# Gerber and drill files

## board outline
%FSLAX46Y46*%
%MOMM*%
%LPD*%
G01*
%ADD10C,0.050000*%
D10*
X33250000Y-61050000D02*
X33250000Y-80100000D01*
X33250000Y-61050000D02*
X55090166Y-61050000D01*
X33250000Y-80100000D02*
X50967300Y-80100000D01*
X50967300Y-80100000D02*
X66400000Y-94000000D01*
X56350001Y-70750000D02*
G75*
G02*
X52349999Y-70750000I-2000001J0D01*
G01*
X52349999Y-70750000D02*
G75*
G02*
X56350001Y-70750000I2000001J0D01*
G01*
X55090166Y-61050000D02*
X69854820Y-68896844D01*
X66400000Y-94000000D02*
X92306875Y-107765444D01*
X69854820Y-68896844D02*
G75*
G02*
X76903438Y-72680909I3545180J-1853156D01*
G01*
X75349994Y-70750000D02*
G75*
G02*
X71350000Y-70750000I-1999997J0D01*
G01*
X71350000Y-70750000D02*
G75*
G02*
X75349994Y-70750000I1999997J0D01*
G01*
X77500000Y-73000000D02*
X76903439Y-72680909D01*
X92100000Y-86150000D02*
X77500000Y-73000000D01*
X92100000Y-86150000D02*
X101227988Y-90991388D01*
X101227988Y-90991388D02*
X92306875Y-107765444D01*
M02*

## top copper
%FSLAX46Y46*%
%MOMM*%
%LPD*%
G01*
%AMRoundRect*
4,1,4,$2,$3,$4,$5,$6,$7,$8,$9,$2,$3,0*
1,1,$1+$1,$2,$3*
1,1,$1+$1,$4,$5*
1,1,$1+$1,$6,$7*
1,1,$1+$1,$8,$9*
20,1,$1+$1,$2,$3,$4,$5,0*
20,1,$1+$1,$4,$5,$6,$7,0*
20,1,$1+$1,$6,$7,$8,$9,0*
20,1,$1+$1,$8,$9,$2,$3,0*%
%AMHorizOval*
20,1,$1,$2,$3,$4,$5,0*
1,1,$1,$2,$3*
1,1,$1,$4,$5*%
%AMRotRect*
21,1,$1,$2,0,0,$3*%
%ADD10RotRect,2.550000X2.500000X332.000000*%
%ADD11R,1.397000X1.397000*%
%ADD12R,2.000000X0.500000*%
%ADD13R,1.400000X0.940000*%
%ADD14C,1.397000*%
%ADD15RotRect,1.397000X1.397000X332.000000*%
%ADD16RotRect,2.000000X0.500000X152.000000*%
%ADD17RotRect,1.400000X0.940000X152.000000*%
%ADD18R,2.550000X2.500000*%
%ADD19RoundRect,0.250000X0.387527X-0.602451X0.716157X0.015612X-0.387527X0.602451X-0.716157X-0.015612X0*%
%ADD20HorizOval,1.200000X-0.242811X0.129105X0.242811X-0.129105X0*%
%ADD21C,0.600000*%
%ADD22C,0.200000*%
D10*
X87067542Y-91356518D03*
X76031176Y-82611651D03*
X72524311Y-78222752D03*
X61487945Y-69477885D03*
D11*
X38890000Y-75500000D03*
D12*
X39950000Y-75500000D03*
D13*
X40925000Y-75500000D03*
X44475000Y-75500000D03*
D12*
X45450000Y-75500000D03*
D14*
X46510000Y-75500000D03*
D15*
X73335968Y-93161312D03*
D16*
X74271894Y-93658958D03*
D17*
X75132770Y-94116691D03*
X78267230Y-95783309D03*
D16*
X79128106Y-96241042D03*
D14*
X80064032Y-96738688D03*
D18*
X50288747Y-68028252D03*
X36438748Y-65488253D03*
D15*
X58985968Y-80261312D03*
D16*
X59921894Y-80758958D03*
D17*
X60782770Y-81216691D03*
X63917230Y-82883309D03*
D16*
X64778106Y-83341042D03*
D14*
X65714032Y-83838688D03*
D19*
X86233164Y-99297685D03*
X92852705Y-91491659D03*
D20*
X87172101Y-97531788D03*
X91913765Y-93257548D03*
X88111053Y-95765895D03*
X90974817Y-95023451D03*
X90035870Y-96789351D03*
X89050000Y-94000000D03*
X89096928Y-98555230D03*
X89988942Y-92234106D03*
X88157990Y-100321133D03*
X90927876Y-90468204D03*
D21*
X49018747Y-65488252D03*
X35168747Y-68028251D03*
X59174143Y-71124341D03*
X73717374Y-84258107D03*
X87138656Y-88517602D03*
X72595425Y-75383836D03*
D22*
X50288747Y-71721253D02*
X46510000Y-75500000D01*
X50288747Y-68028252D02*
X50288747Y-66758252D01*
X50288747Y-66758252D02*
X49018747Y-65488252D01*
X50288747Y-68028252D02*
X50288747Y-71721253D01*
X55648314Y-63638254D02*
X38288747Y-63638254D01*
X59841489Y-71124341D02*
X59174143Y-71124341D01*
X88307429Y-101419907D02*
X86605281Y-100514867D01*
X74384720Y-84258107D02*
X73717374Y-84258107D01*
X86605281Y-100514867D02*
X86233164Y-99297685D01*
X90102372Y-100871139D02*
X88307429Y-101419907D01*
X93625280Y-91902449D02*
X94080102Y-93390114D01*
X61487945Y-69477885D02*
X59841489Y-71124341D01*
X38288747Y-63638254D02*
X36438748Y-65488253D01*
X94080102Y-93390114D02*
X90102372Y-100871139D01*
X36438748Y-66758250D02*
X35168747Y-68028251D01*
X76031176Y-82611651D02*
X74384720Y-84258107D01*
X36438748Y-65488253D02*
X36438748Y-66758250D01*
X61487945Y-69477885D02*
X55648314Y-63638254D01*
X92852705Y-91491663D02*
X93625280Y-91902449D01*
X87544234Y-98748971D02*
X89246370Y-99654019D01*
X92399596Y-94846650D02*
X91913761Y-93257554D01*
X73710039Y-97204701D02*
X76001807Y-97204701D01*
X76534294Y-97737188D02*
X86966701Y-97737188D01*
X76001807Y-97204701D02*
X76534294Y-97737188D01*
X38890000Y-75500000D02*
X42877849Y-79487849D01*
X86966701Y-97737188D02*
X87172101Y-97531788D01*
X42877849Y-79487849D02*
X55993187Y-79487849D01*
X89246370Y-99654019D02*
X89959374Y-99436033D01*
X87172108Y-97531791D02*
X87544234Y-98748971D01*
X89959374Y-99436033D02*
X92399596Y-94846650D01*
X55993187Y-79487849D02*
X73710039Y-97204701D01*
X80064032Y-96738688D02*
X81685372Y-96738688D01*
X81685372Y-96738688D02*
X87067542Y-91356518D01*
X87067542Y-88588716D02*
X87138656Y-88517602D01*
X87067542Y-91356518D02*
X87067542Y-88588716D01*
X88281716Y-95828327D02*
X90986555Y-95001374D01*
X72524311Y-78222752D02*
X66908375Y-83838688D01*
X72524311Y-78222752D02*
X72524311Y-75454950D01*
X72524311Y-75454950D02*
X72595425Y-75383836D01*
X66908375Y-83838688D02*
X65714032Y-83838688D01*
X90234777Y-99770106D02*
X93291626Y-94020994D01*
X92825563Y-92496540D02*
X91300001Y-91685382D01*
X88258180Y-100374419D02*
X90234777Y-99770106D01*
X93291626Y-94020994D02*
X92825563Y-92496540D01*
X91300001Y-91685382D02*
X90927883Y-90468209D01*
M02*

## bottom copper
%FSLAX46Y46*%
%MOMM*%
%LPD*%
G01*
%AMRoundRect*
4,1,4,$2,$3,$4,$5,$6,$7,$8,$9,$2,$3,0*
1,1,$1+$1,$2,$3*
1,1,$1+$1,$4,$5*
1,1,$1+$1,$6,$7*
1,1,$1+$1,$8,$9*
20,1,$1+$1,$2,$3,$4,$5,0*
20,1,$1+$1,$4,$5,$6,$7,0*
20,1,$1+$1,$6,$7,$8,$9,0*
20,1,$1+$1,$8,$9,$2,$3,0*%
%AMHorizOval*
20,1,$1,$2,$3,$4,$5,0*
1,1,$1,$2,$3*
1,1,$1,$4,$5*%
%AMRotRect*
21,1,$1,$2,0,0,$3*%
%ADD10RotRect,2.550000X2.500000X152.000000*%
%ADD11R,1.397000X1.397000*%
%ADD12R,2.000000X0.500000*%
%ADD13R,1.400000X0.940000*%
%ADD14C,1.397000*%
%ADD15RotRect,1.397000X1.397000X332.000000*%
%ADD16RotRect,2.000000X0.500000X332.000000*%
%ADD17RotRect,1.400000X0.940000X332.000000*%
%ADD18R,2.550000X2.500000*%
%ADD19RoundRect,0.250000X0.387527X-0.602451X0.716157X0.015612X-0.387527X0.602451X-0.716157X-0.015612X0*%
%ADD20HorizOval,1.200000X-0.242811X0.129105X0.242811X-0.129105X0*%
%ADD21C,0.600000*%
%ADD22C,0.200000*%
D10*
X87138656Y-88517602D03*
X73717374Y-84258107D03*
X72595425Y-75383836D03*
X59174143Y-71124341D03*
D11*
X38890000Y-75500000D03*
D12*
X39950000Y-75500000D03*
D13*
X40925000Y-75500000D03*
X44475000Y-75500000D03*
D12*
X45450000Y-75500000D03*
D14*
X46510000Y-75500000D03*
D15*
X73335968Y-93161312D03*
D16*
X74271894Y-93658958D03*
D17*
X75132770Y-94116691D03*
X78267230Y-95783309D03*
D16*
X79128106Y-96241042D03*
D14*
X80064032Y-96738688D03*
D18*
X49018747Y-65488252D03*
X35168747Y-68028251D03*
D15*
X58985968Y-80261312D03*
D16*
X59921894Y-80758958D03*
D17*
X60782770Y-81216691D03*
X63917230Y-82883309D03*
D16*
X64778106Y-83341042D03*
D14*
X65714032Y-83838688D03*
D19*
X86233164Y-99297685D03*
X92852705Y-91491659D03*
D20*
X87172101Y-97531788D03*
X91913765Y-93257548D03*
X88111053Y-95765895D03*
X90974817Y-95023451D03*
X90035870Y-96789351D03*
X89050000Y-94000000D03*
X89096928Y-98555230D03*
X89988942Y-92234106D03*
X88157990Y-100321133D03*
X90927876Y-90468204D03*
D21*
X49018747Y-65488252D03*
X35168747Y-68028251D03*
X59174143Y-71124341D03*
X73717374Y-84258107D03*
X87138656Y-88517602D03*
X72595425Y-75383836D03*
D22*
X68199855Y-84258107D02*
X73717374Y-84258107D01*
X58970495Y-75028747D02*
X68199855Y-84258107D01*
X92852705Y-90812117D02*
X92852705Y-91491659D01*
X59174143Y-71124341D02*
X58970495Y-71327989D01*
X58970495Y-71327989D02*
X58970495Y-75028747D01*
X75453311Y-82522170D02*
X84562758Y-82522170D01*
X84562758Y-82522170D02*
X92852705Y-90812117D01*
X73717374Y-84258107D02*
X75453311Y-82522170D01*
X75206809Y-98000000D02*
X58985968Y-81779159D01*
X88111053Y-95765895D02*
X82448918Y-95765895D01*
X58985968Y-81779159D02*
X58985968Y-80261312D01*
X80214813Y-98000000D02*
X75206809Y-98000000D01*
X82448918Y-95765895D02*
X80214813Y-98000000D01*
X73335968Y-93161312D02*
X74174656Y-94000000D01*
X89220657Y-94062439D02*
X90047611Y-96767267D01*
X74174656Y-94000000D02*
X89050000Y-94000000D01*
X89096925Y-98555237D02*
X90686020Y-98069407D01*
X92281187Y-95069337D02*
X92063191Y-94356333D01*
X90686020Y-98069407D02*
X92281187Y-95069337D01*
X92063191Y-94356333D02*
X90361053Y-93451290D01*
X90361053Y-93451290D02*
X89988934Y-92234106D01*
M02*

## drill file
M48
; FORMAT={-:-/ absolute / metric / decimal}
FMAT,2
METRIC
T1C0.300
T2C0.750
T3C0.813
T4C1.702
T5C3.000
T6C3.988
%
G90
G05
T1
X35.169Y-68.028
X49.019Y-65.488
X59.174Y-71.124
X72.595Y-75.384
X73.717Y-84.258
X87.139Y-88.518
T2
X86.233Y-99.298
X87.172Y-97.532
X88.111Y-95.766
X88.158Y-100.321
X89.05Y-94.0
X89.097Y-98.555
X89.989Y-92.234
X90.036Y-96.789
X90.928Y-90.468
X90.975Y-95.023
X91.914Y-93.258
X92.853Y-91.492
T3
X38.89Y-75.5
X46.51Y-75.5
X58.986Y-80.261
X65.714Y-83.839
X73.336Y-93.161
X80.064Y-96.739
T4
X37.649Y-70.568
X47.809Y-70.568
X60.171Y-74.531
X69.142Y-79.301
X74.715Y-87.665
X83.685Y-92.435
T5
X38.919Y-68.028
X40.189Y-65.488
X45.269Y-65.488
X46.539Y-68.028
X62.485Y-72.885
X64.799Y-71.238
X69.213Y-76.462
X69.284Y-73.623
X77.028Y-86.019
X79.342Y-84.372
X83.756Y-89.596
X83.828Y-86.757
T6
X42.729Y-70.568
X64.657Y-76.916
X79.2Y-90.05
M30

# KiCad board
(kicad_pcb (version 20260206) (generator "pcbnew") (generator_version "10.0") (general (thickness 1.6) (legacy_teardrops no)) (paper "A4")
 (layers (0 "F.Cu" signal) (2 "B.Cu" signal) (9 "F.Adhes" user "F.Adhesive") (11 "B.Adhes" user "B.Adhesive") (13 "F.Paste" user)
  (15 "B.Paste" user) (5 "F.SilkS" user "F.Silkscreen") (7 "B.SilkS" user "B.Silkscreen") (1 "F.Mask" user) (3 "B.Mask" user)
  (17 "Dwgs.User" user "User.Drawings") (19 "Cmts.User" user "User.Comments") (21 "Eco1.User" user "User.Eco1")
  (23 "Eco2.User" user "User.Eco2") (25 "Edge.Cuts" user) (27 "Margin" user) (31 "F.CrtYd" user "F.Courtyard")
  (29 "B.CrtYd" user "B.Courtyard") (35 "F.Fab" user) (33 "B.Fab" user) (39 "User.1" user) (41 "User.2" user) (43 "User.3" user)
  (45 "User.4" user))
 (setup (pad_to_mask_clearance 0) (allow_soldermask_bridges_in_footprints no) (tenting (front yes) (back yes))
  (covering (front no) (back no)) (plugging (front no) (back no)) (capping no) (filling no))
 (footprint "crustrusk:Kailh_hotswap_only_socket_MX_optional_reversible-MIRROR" (layer "F.Cu") (at 79.2 90.05 -28)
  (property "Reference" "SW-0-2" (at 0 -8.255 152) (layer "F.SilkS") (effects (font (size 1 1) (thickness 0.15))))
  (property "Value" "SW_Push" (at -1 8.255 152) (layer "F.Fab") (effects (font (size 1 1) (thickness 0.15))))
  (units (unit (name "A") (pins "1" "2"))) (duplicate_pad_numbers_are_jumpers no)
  (pad "" np_thru_hole circle (at -5.08 0 332) (size 1.7018 1.7018) (drill 1.7018) (layers "*.Cu" "*.Mask"))
  (pad "" np_thru_hole circle (at -3.810001 -2.54 152) (size 3 3) (drill 3) (layers "*.Cu" "*.Mask"))
  (pad "" np_thru_hole circle (at -2.54 -5.079998 332) (size 3 3) (drill 3) (layers "*.Cu" "*.Mask"))
  (pad "" np_thru_hole circle (at 0 0 332) (size 3.9878 3.9878) (drill 3.9878) (layers "*.Cu" "*.Mask"))
  (pad "" np_thru_hole circle (at 2.540002 -5.080001 152) (size 3 3) (drill 3) (layers "*.Cu" "*.Mask"))
  (pad "" np_thru_hole circle (at 3.81 -2.54 332) (size 3 3) (drill 3) (layers "*.Cu" "*.Mask"))
  (pad "" np_thru_hole circle (at 5.08 0 332) (size 1.7018 1.7018) (drill 1.7018) (layers "*.Cu" "*.Mask"))
  (pad "1" smd rect (at 6.29 -5.08 152) (size 2.55 2.5) (layers "B.Cu" "B.Mask" "B.Paste") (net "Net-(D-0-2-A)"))
  (pad "1" smd rect (at 7.56 -2.54 332) (size 2.55 2.5) (layers "F.Cu" "F.Mask" "F.Paste") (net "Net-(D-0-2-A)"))
  (pad "2" smd rect (at -7.56 -2.540001 152) (size 2.55 2.5) (layers "B.Cu" "B.Mask" "B.Paste") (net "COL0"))
  (pad "2" smd rect (at -6.289999 -5.08 332) (size 2.55 2.5) (layers "F.Cu" "F.Mask" "F.Paste") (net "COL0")))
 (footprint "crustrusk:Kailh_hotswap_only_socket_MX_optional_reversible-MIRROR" (layer "F.Cu") (at 64.656769 76.916234 -28)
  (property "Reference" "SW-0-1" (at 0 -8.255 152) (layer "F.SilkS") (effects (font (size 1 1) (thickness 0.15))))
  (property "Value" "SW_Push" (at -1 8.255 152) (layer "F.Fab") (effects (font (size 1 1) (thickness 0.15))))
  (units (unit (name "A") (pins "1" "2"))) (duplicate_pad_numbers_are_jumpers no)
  (pad "" np_thru_hole circle (at -5.08 0 332) (size 1.7018 1.7018) (drill 1.7018) (layers "*.Cu" "*.Mask"))
  (pad "" np_thru_hole circle (at -3.810001 -2.54 152) (size 3 3) (drill 3) (layers "*.Cu" "*.Mask"))
  (pad "" np_thru_hole circle (at -2.54 -5.079998 332) (size 3 3) (drill 3) (layers "*.Cu" "*.Mask"))
  (pad "" np_thru_hole circle (at 0 0 332) (size 3.9878 3.9878) (drill 3.9878) (layers "*.Cu" "*.Mask"))
  (pad "" np_thru_hole circle (at 2.540002 -5.080001 152) (size 3 3) (drill 3) (layers "*.Cu" "*.Mask"))
  (pad "" np_thru_hole circle (at 3.81 -2.54 332) (size 3 3) (drill 3) (layers "*.Cu" "*.Mask"))
  (pad "" np_thru_hole circle (at 5.08 0 332) (size 1.7018 1.7018) (drill 1.7018) (layers "*.Cu" "*.Mask"))
  (pad "1" smd rect (at 6.29 -5.08 152) (size 2.55 2.5) (layers "B.Cu" "B.Mask" "B.Paste") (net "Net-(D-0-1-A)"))
  (pad "1" smd rect (at 7.56 -2.54 332) (size 2.55 2.5) (layers "F.Cu" "F.Mask" "F.Paste") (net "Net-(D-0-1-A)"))
  (pad "2" smd rect (at -7.56 -2.540001 152) (size 2.55 2.5) (layers "B.Cu" "B.Mask" "B.Paste") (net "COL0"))
  (pad "2" smd rect (at -6.289999 -5.08 332) (size 2.55 2.5) (layers "F.Cu" "F.Mask" "F.Paste") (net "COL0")))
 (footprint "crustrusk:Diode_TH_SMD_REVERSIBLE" (layer "F.Cu") (at 42.7 75.5)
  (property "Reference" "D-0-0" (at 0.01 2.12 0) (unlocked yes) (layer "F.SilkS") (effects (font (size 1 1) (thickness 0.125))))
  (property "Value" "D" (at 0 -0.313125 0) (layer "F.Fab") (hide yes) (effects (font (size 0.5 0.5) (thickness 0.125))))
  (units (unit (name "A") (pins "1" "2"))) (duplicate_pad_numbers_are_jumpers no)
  (pad "1" thru_hole rect (at -3.81 0) (size 1.397 1.397) (drill 0.8128) (layers "*.Cu" "*.Mask") (remove_unused_layers no) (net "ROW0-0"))
  (pad "1" smd rect (at -2.75 0 180) (size 2 0.5) (layers "F.Cu") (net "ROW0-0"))
  (pad "1" smd rect (at -2.75 0) (size 2 0.5) (layers "B.Cu") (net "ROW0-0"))
  (pad "1" smd rect (at -1.775 0 180) (size 1.4 0.94) (layers "F.Cu" "F.Mask" "F.Paste") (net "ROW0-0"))
  (pad "1" smd rect (at -1.775 0) (size 1.4 0.94) (layers "B.Cu" "B.Mask" "B.Paste") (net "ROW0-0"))
  (pad "2" smd rect (at 1.775 0 180) (size 1.4 0.94) (layers "F.Cu" "F.Mask" "F.Paste") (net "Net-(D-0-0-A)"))
  (pad "2" smd rect (at 1.775 0) (size 1.4 0.94) (layers "B.Cu" "B.Mask" "B.Paste") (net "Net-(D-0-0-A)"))
  (pad "2" smd rect (at 2.75 0 180) (size 2 0.5) (layers "F.Cu") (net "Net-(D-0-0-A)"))
  (pad "2" smd rect (at 2.75 0) (size 2 0.5) (layers "B.Cu") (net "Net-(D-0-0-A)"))
  (pad "2" thru_hole circle (at 3.81 0) (size 1.397 1.397) (drill 0.8128) (layers "*.Cu" "*.Mask") (remove_unused_layers no)
   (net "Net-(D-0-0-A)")))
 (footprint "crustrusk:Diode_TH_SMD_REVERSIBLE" (layer "F.Cu") (at 76.7 94.95 -28)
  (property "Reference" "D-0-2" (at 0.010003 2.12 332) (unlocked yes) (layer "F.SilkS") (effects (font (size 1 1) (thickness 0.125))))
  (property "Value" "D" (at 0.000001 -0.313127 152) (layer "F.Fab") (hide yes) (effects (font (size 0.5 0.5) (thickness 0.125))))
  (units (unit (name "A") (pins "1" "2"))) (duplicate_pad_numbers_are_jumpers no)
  (pad "1" thru_hole rect (at -3.810002 0 332) (size 1.397 1.397) (drill 0.8128) (layers "*.Cu" "*.Mask") (remove_unused_layers no)
   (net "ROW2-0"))
  (pad "1" smd rect (at -2.749998 0.000004 152) (size 2 0.5) (layers "F.Cu") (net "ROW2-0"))
  (pad "1" smd rect (at -2.749998 0.000004 332) (size 2 0.5) (layers "B.Cu") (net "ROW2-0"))
  (pad "1" smd rect (at -1.774997 0.000002 152) (size 1.4 0.94) (layers "F.Cu" "F.Mask" "F.Paste") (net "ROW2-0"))
  (pad "1" smd rect (at -1.774997 0.000002 332) (size 1.4 0.94) (layers "B.Cu" "B.Mask" "B.Paste") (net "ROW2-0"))
  (pad "2" smd rect (at 1.774997 -0.000002 152) (size 1.4 0.94) (layers "F.Cu" "F.Mask" "F.Paste") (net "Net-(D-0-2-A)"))
  (pad "2" smd rect (at 1.774997 -0.000002 332) (size 1.4 0.94) (layers "B.Cu" "B.Mask" "B.Paste") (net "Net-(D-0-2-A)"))
  (pad "2" smd rect (at 2.749998 -0.000004 152) (size 2 0.5) (layers "F.Cu") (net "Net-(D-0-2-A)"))
  (pad "2" smd rect (at 2.749998 -0.000004 332) (size 2 0.5) (layers "B.Cu") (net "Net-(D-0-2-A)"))
  (pad "2" thru_hole circle (at 3.810002 0 332) (size 1.397 1.397) (drill 0.8128) (layers "*.Cu" "*.Mask") (remove_unused_layers no)
   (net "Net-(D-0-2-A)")))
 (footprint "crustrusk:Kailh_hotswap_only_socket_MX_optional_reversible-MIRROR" (layer "F.Cu") (at 42.728747 70.568252)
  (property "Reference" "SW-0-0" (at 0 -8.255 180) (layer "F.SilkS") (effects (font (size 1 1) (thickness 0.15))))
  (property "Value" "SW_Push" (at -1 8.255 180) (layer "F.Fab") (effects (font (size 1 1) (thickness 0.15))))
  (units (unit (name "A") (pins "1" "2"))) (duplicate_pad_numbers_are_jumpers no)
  (pad "" np_thru_hole circle (at -5.08 0) (size 1.7018 1.7018) (drill 1.7018) (layers "*.Cu" "*.Mask"))
  (pad "" np_thru_hole circle (at -3.81 -2.54 180) (size 3 3) (drill 3) (layers "*.Cu" "*.Mask"))
  (pad "" np_thru_hole circle (at -2.54 -5.079998) (size 3 3) (drill 3) (layers "*.Cu" "*.Mask"))
  (pad "" np_thru_hole circle (at 0 0) (size 3.9878 3.9878) (drill 3.9878) (layers "*.Cu" "*.Mask"))
  (pad "" np_thru_hole circle (at 2.540002 -5.080001 180) (size 3 3) (drill 3) (layers "*.Cu" "*.Mask"))
  (pad "" np_thru_hole circle (at 3.81 -2.54) (size 3 3) (drill 3) (layers "*.Cu" "*.Mask"))
  (pad "" np_thru_hole circle (at 5.08 0) (size 1.7018 1.7018) (drill 1.7018) (layers "*.Cu" "*.Mask"))
  (pad "1" smd rect (at 6.29 -5.08 180) (size 2.55 2.5) (layers "B.Cu" "B.Mask" "B.Paste") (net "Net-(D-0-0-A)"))
  (pad "1" smd rect (at 7.56 -2.54) (size 2.55 2.5) (layers "F.Cu" "F.Mask" "F.Paste") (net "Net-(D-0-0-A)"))
  (pad "2" smd rect (at -7.56 -2.540001 180) (size 2.55 2.5) (layers "B.Cu" "B.Mask" "B.Paste") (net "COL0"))
  (pad "2" smd rect (at -6.289999 -5.079999) (size 2.55 2.5) (layers "F.Cu" "F.Mask" "F.Paste") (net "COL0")))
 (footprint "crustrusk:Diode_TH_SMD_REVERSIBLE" (layer "F.Cu") (at 62.35 82.05 -28)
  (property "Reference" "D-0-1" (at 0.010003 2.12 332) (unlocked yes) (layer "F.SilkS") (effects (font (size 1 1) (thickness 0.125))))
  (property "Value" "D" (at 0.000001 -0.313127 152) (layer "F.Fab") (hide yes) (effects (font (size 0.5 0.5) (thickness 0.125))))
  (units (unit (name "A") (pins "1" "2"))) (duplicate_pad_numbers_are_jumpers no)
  (pad "1" thru_hole rect (at -3.810002 0 332) (size 1.397 1.397) (drill 0.8128) (layers "*.Cu" "*.Mask") (remove_unused_layers no)
   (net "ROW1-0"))
  (pad "1" smd rect (at -2.749998 0.000004 152) (size 2 0.5) (layers "F.Cu") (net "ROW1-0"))
  (pad "1" smd rect (at -2.749998 0.000004 332) (size 2 0.5) (layers "B.Cu") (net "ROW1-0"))
  (pad "1" smd rect (at -1.774997 0.000002 152) (size 1.4 0.94) (layers "F.Cu" "F.Mask" "F.Paste") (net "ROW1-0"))
  (pad "1" smd rect (at -1.774997 0.000002 332) (size 1.4 0.94) (layers "B.Cu" "B.Mask" "B.Paste") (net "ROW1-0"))
  (pad "2" smd rect (at 1.774997 -0.000002 152) (size 1.4 0.94) (layers "F.Cu" "F.Mask" "F.Paste") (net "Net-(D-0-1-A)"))
  (pad "2" smd rect (at 1.774997 -0.000002 332) (size 1.4 0.94) (layers "B.Cu" "B.Mask" "B.Paste") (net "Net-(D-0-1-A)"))
  (pad "2" smd rect (at 2.749998 -0.000004 152) (size 2 0.5) (layers "F.Cu") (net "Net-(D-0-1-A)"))
  (pad "2" smd rect (at 2.749998 -0.000004 332) (size 2 0.5) (layers "B.Cu") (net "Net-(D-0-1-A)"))
  (pad "2" thru_hole circle (at 3.810002 0 332) (size 1.397 1.397) (drill 0.8128) (layers "*.Cu" "*.Mask") (remove_unused_layers no)
   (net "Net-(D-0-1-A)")))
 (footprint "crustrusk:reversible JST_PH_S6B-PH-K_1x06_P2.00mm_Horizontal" (layer "F.Cu") (at 86.233164 99.297685 62)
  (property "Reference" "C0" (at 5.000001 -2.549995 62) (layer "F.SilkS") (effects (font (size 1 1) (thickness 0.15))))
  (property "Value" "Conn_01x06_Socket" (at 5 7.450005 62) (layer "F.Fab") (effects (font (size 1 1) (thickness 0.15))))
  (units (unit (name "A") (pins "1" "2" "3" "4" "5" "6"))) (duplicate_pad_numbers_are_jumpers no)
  (pad "1" thru_hole roundrect (at 0 0 62) (size 1.2 1.75) (drill 0.75) (layers "*.Cu" "*.Mask") (remove_unused_layers no)
   (roundrect_rratio 0.208333) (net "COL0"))
  (pad "1" thru_hole roundrect (at 9.999998 2.180001 62) (size 1.2 1.75) (drill 0.75) (layers "*.Cu" "*.Mask") (remove_unused_layers no)
   (roundrect_rratio 0.208333) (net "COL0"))
  (pad "2" thru_hole oval (at 1.999999 -0.000006 62) (size 1.2 1.75) (drill 0.75) (layers "*.Cu" "*.Mask") (remove_unused_layers no)
   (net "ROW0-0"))
  (pad "2" thru_hole oval (at 8.000005 2.18 62) (size 1.2 1.75) (drill 0.75) (layers "*.Cu" "*.Mask") (remove_unused_layers no)
   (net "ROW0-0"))
  (pad "3" thru_hole oval (at 4.000001 0.000003 62) (size 1.2 1.75) (drill 0.75) (layers "*.Cu" "*.Mask") (remove_unused_layers no)
   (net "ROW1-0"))
  (pad "3" thru_hole oval (at 5.999996 2.18 62) (size 1.2 1.75) (drill 0.75) (layers "*.Cu" "*.Mask") (remove_unused_layers no)
   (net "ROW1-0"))
  (pad "4" thru_hole oval (at 3.99999 2.179999 62) (size 1.2 1.75) (drill 0.75) (layers "*.Cu" "*.Mask") (remove_unused_layers no)
   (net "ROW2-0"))
  (pad "4" thru_hole oval (at 6.000003 0.000006 62) (size 1.2 1.75) (drill 0.75) (layers "*.Cu" "*.Mask") (remove_unused_layers no)
   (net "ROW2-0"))
  (pad "5" thru_hole oval (at 2.000005 2.179992 62) (size 1.2 1.75) (drill 0.75) (layers "*.Cu" "*.Mask") (remove_unused_layers no)
   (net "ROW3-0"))
  (pad "5" thru_hole oval (at 8.000001 0.000006 62) (size 1.2 1.75) (drill 0.75) (layers "*.Cu" "*.Mask") (remove_unused_layers no)
   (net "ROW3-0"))
  (pad "6" thru_hole oval (at 0 2.18 62) (size 1.2 1.75) (drill 0.75) (layers "*.Cu" "*.Mask") (remove_unused_layers no) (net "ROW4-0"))
  (pad "6" thru_hole oval (at 10.000003 -0.000006 62) (size 1.2 1.75) (drill 0.75) (layers "*.Cu" "*.Mask") (remove_unused_layers no)
   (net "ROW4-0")))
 (gr_line (start 33.25 61.05) (end 33.25 80.1) (stroke (width 0.05) (type default)) (layer "Edge.Cuts"))
 (gr_line (start 33.25 61.05) (end 55.090166 61.05) (stroke (width 0.05) (type default)) (layer "Edge.Cuts"))
 (gr_line (start 33.25 80.1) (end 50.9673 80.1) (stroke (width 0.05) (type default)) (layer "Edge.Cuts"))
 (gr_line (start 50.9673 80.1) (end 66.4 94) (stroke (width 0.05) (type default)) (layer "Edge.Cuts"))
 (gr_circle (center 54.35 70.75) (end 52.349999 70.75) (stroke (width 0.05) (type default)) (fill no) (layer "Edge.Cuts"))
 (gr_line (start 55.090166 61.05) (end 69.85482 68.896844) (stroke (width 0.05) (type default)) (layer "Edge.Cuts"))
 (gr_line (start 66.4 94) (end 92.306875 107.765444) (stroke (width 0.05) (type default)) (layer "Edge.Cuts"))
 (gr_arc (start 69.85482 68.896844) (mid 75.292148 67.225477) (end 76.903438 72.680909) (stroke (width 0.05) (type default))
  (layer "Edge.Cuts"))
 (gr_circle (center 73.349997 70.75) (end 71.35 70.75) (stroke (width 0.05) (type default)) (fill no) (layer "Edge.Cuts"))
 (gr_line (start 77.5 73) (end 76.903439 72.680909) (stroke (width 0.05) (type default)) (layer "Edge.Cuts"))
 (gr_line (start 92.1 86.15) (end 77.5 73) (stroke (width 0.05) (type default)) (layer "Edge.Cuts"))
 (gr_line (start 92.1 86.15) (end 101.227988 90.991388) (stroke (width 0.05) (type default)) (layer "Edge.Cuts"))
 (gr_line (start 101.227988 90.991388) (end 92.306875 107.765444) (stroke (width 0.05) (type default)) (layer "Edge.Cuts"))
 (segment (start 50.288747 71.721253) (end 46.51 75.5) (width 0.2) (layer "F.Cu") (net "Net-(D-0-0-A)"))
 (segment (start 50.288747 68.028252) (end 50.288747 66.758252) (width 0.2) (layer "F.Cu") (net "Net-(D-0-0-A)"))
 (segment (start 50.288747 66.758252) (end 49.018747 65.488252) (width 0.2) (layer "F.Cu") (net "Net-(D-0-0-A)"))
 (segment (start 50.288747 68.028252) (end 50.288747 71.721253) (width 0.2) (layer "F.Cu") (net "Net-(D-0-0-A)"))
 (via (at 49.018747 65.488252) (size 0.6) (drill 0.3) (layers "F.Cu" "B.Cu") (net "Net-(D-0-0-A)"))
 (segment (start 55.648314 63.638254) (end 38.288747 63.638254) (width 0.2) (layer "F.Cu") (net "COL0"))
 (segment (start 59.841489 71.124341) (end 59.174143 71.124341) (width 0.2) (layer "F.Cu") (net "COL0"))
 (segment (start 88.307429 101.419907) (end 86.605281 100.514867) (width 0.2) (layer "F.Cu") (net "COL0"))
 (segment (start 74.38472 84.258107) (end 73.717374 84.258107) (width 0.2) (layer "F.Cu") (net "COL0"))
 (segment (start 86.605281 100.514867) (end 86.233164 99.297685) (width 0.2) (layer "F.Cu") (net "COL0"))
 (segment (start 90.102372 100.871139) (end 88.307429 101.419907) (width 0.2) (layer "F.Cu") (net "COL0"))
 (segment (start 93.62528 91.902449) (end 94.080102 93.390114) (width 0.2) (layer "F.Cu") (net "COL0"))
 (segment (start 61.487945 69.477885) (end 59.841489 71.124341) (width 0.2) (layer "F.Cu") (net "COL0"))
 (segment (start 38.288747 63.638254) (end 36.438748 65.488253) (width 0.2) (layer "F.Cu") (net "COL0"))
 (segment (start 94.080102 93.390114) (end 90.102372 100.871139) (width 0.2) (layer "F.Cu") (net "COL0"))
 (segment (start 36.438748 66.75825) (end 35.168747 68.028251) (width 0.2) (layer "F.Cu") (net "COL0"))
 (segment (start 76.031176 82.611651) (end 74.38472 84.258107) (width 0.2) (layer "F.Cu") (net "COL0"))
 (segment (start 36.438748 65.488253) (end 36.438748 66.75825) (width 0.2) (layer "F.Cu") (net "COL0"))
 (segment (start 61.487945 69.477885) (end 55.648314 63.638254) (width 0.2) (layer "F.Cu") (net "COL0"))
 (segment (start 92.852705 91.491663) (end 93.62528 91.902449) (width 0.2) (layer "F.Cu") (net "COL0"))
 (via (at 35.168747 68.028251) (size 0.6) (drill 0.3) (layers "F.Cu" "B.Cu") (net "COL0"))
 (via (at 59.174143 71.124341) (size 0.6) (drill 0.3) (layers "F.Cu" "B.Cu") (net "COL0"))
 (via (at 73.717374 84.258107) (size 0.6) (drill 0.3) (layers "F.Cu" "B.Cu") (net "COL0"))
 (segment (start 68.199855 84.258107) (end 73.717374 84.258107) (width 0.2) (layer "B.Cu") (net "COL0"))
 (segment (start 58.970495 75.028747) (end 68.199855 84.258107) (width 0.2) (layer "B.Cu") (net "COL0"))
 (segment (start 92.852705 90.812117) (end 92.852705 91.491659) (width 0.2) (layer "B.Cu") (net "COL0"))
 (segment (start 59.174143 71.124341) (end 58.970495 71.327989) (width 0.2) (layer "B.Cu") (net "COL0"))
 (segment (start 58.970495 71.327989) (end 58.970495 75.028747) (width 0.2) (layer "B.Cu") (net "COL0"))
 (segment (start 75.453311 82.52217) (end 84.562758 82.52217) (width 0.2) (layer "B.Cu") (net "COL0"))
 (segment (start 84.562758 82.52217) (end 92.852705 90.812117) (width 0.2) (layer "B.Cu") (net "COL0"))
 (segment (start 73.717374 84.258107) (end 75.453311 82.52217) (width 0.2) (layer "B.Cu") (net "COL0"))
 (segment (start 87.544234 98.748971) (end 89.24637 99.654019) (width 0.2) (layer "F.Cu") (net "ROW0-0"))
 (segment (start 92.399596 94.84665) (end 91.913761 93.257554) (width 0.2) (layer "F.Cu") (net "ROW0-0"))
 (segment (start 73.710039 97.204701) (end 76.001807 97.204701) (width 0.2) (layer "F.Cu") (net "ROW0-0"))
 (segment (start 76.534294 97.737188) (end 86.966701 97.737188) (width 0.2) (layer "F.Cu") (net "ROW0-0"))
 (segment (start 76.001807 97.204701) (end 76.534294 97.737188) (width 0.2) (layer "F.Cu") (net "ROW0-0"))
 (segment (start 38.89 75.5) (end 42.877849 79.487849) (width 0.2) (layer "F.Cu") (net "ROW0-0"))
 (segment (start 86.966701 97.737188) (end 87.172101 97.531788) (width 0.2) (layer "F.Cu") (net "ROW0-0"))
 (segment (start 42.877849 79.487849) (end 55.993187 79.487849) (width 0.2) (layer "F.Cu") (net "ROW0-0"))
 (segment (start 89.24637 99.654019) (end 89.959374 99.436033) (width 0.2) (layer "F.Cu") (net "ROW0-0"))
 (segment (start 87.172108 97.531791) (end 87.544234 98.748971) (width 0.2) (layer "F.Cu") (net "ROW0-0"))
 (segment (start 89.959374 99.436033) (end 92.399596 94.84665) (width 0.2) (layer "F.Cu") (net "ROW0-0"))
 (segment (start 55.993187 79.487849) (end 73.710039 97.204701) (width 0.2) (layer "F.Cu") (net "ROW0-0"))
 (segment (start 80.064032 96.738688) (end 81.685372 96.738688) (width 0.2) (layer "F.Cu") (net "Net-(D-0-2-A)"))
 (segment (start 81.685372 96.738688) (end 87.067542 91.356518) (width 0.2) (layer "F.Cu") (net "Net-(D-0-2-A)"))
 (segment (start 87.067542 88.588716) (end 87.138656 88.517602) (width 0.2) (layer "F.Cu") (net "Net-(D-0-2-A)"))
 (segment (start 87.067542 91.356518) (end 87.067542 88.588716) (width 0.2) (layer "F.Cu") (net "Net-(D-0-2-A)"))
 (via (at 87.138656 88.517602) (size 0.6) (drill 0.3) (layers "F.Cu" "B.Cu") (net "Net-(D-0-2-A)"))
 (segment (start 88.281716 95.828327) (end 90.986555 95.001374) (width 0.2) (layer "F.Cu") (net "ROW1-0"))
 (segment (start 75.206809 98) (end 58.985968 81.779159) (width 0.2) (layer "B.Cu") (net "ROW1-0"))
 (segment (start 88.111053 95.765895) (end 82.448918 95.765895) (width 0.2) (layer "B.Cu") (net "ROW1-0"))
 (segment (start 58.985968 81.779159) (end 58.985968 80.261312) (width 0.2) (layer "B.Cu") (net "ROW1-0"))
 (segment (start 80.214813 98) (end 75.206809 98) (width 0.2) (layer "B.Cu") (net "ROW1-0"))
 (segment (start 82.448918 95.765895) (end 80.214813 98) (width 0.2) (layer "B.Cu") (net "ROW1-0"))
 (segment (start 72.524311 78.222752) (end 66.908375 83.838688) (width 0.2) (layer "F.Cu") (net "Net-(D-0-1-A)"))
 (segment (start 72.524311 78.222752) (end 72.524311 75.45495) (width 0.2) (layer "F.Cu") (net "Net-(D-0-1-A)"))
 (segment (start 72.524311 75.45495) (end 72.595425 75.383836) (width 0.2) (layer "F.Cu") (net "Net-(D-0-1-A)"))
 (segment (start 66.908375 83.838688) (end 65.714032 83.838688) (width 0.2) (layer "F.Cu") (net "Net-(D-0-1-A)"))
 (via (at 72.595425 75.383836) (size 0.6) (drill 0.3) (layers "F.Cu" "B.Cu") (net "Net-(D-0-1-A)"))
 (segment (start 73.335968 93.161312) (end 74.174656 94) (width 0.2) (layer "B.Cu") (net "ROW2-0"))
 (segment (start 89.220657 94.062439) (end 90.047611 96.767267) (width 0.2) (layer "B.Cu") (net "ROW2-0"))
 (segment (start 74.174656 94) (end 89.05 94) (width 0.2) (layer "B.Cu") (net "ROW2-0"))
 (segment (start 89.096925 98.555237) (end 90.68602 98.069407) (width 0.2) (layer "B.Cu") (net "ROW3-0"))
 (segment (start 92.281187 95.069337) (end 92.063191 94.356333) (width 0.2) (layer "B.Cu") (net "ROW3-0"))
 (segment (start 90.68602 98.069407) (end 92.281187 95.069337) (width 0.2) (layer "B.Cu") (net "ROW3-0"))
 (segment (start 92.063191 94.356333) (end 90.361053 93.45129) (width 0.2) (layer "B.Cu") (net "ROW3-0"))
 (segment (start 90.361053 93.45129) (end 89.988934 92.234106) (width 0.2) (layer "B.Cu") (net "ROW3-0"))
 (segment (start 90.234777 99.770106) (end 93.291626 94.020994) (width 0.2) (layer "F.Cu") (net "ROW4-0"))
 (segment (start 92.825563 92.49654) (end 91.300001 91.685382) (width 0.2) (layer "F.Cu") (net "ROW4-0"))
 (segment (start 88.25818 100.374419) (end 90.234777 99.770106) (width 0.2) (layer "F.Cu") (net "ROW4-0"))
 (segment (start 93.291626 94.020994) (end 92.825563 92.49654) (width 0.2) (layer "F.Cu") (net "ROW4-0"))
 (segment (start 91.300001 91.685382) (end 90.927883 90.468209) (width 0.2) (layer "F.Cu") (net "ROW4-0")))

